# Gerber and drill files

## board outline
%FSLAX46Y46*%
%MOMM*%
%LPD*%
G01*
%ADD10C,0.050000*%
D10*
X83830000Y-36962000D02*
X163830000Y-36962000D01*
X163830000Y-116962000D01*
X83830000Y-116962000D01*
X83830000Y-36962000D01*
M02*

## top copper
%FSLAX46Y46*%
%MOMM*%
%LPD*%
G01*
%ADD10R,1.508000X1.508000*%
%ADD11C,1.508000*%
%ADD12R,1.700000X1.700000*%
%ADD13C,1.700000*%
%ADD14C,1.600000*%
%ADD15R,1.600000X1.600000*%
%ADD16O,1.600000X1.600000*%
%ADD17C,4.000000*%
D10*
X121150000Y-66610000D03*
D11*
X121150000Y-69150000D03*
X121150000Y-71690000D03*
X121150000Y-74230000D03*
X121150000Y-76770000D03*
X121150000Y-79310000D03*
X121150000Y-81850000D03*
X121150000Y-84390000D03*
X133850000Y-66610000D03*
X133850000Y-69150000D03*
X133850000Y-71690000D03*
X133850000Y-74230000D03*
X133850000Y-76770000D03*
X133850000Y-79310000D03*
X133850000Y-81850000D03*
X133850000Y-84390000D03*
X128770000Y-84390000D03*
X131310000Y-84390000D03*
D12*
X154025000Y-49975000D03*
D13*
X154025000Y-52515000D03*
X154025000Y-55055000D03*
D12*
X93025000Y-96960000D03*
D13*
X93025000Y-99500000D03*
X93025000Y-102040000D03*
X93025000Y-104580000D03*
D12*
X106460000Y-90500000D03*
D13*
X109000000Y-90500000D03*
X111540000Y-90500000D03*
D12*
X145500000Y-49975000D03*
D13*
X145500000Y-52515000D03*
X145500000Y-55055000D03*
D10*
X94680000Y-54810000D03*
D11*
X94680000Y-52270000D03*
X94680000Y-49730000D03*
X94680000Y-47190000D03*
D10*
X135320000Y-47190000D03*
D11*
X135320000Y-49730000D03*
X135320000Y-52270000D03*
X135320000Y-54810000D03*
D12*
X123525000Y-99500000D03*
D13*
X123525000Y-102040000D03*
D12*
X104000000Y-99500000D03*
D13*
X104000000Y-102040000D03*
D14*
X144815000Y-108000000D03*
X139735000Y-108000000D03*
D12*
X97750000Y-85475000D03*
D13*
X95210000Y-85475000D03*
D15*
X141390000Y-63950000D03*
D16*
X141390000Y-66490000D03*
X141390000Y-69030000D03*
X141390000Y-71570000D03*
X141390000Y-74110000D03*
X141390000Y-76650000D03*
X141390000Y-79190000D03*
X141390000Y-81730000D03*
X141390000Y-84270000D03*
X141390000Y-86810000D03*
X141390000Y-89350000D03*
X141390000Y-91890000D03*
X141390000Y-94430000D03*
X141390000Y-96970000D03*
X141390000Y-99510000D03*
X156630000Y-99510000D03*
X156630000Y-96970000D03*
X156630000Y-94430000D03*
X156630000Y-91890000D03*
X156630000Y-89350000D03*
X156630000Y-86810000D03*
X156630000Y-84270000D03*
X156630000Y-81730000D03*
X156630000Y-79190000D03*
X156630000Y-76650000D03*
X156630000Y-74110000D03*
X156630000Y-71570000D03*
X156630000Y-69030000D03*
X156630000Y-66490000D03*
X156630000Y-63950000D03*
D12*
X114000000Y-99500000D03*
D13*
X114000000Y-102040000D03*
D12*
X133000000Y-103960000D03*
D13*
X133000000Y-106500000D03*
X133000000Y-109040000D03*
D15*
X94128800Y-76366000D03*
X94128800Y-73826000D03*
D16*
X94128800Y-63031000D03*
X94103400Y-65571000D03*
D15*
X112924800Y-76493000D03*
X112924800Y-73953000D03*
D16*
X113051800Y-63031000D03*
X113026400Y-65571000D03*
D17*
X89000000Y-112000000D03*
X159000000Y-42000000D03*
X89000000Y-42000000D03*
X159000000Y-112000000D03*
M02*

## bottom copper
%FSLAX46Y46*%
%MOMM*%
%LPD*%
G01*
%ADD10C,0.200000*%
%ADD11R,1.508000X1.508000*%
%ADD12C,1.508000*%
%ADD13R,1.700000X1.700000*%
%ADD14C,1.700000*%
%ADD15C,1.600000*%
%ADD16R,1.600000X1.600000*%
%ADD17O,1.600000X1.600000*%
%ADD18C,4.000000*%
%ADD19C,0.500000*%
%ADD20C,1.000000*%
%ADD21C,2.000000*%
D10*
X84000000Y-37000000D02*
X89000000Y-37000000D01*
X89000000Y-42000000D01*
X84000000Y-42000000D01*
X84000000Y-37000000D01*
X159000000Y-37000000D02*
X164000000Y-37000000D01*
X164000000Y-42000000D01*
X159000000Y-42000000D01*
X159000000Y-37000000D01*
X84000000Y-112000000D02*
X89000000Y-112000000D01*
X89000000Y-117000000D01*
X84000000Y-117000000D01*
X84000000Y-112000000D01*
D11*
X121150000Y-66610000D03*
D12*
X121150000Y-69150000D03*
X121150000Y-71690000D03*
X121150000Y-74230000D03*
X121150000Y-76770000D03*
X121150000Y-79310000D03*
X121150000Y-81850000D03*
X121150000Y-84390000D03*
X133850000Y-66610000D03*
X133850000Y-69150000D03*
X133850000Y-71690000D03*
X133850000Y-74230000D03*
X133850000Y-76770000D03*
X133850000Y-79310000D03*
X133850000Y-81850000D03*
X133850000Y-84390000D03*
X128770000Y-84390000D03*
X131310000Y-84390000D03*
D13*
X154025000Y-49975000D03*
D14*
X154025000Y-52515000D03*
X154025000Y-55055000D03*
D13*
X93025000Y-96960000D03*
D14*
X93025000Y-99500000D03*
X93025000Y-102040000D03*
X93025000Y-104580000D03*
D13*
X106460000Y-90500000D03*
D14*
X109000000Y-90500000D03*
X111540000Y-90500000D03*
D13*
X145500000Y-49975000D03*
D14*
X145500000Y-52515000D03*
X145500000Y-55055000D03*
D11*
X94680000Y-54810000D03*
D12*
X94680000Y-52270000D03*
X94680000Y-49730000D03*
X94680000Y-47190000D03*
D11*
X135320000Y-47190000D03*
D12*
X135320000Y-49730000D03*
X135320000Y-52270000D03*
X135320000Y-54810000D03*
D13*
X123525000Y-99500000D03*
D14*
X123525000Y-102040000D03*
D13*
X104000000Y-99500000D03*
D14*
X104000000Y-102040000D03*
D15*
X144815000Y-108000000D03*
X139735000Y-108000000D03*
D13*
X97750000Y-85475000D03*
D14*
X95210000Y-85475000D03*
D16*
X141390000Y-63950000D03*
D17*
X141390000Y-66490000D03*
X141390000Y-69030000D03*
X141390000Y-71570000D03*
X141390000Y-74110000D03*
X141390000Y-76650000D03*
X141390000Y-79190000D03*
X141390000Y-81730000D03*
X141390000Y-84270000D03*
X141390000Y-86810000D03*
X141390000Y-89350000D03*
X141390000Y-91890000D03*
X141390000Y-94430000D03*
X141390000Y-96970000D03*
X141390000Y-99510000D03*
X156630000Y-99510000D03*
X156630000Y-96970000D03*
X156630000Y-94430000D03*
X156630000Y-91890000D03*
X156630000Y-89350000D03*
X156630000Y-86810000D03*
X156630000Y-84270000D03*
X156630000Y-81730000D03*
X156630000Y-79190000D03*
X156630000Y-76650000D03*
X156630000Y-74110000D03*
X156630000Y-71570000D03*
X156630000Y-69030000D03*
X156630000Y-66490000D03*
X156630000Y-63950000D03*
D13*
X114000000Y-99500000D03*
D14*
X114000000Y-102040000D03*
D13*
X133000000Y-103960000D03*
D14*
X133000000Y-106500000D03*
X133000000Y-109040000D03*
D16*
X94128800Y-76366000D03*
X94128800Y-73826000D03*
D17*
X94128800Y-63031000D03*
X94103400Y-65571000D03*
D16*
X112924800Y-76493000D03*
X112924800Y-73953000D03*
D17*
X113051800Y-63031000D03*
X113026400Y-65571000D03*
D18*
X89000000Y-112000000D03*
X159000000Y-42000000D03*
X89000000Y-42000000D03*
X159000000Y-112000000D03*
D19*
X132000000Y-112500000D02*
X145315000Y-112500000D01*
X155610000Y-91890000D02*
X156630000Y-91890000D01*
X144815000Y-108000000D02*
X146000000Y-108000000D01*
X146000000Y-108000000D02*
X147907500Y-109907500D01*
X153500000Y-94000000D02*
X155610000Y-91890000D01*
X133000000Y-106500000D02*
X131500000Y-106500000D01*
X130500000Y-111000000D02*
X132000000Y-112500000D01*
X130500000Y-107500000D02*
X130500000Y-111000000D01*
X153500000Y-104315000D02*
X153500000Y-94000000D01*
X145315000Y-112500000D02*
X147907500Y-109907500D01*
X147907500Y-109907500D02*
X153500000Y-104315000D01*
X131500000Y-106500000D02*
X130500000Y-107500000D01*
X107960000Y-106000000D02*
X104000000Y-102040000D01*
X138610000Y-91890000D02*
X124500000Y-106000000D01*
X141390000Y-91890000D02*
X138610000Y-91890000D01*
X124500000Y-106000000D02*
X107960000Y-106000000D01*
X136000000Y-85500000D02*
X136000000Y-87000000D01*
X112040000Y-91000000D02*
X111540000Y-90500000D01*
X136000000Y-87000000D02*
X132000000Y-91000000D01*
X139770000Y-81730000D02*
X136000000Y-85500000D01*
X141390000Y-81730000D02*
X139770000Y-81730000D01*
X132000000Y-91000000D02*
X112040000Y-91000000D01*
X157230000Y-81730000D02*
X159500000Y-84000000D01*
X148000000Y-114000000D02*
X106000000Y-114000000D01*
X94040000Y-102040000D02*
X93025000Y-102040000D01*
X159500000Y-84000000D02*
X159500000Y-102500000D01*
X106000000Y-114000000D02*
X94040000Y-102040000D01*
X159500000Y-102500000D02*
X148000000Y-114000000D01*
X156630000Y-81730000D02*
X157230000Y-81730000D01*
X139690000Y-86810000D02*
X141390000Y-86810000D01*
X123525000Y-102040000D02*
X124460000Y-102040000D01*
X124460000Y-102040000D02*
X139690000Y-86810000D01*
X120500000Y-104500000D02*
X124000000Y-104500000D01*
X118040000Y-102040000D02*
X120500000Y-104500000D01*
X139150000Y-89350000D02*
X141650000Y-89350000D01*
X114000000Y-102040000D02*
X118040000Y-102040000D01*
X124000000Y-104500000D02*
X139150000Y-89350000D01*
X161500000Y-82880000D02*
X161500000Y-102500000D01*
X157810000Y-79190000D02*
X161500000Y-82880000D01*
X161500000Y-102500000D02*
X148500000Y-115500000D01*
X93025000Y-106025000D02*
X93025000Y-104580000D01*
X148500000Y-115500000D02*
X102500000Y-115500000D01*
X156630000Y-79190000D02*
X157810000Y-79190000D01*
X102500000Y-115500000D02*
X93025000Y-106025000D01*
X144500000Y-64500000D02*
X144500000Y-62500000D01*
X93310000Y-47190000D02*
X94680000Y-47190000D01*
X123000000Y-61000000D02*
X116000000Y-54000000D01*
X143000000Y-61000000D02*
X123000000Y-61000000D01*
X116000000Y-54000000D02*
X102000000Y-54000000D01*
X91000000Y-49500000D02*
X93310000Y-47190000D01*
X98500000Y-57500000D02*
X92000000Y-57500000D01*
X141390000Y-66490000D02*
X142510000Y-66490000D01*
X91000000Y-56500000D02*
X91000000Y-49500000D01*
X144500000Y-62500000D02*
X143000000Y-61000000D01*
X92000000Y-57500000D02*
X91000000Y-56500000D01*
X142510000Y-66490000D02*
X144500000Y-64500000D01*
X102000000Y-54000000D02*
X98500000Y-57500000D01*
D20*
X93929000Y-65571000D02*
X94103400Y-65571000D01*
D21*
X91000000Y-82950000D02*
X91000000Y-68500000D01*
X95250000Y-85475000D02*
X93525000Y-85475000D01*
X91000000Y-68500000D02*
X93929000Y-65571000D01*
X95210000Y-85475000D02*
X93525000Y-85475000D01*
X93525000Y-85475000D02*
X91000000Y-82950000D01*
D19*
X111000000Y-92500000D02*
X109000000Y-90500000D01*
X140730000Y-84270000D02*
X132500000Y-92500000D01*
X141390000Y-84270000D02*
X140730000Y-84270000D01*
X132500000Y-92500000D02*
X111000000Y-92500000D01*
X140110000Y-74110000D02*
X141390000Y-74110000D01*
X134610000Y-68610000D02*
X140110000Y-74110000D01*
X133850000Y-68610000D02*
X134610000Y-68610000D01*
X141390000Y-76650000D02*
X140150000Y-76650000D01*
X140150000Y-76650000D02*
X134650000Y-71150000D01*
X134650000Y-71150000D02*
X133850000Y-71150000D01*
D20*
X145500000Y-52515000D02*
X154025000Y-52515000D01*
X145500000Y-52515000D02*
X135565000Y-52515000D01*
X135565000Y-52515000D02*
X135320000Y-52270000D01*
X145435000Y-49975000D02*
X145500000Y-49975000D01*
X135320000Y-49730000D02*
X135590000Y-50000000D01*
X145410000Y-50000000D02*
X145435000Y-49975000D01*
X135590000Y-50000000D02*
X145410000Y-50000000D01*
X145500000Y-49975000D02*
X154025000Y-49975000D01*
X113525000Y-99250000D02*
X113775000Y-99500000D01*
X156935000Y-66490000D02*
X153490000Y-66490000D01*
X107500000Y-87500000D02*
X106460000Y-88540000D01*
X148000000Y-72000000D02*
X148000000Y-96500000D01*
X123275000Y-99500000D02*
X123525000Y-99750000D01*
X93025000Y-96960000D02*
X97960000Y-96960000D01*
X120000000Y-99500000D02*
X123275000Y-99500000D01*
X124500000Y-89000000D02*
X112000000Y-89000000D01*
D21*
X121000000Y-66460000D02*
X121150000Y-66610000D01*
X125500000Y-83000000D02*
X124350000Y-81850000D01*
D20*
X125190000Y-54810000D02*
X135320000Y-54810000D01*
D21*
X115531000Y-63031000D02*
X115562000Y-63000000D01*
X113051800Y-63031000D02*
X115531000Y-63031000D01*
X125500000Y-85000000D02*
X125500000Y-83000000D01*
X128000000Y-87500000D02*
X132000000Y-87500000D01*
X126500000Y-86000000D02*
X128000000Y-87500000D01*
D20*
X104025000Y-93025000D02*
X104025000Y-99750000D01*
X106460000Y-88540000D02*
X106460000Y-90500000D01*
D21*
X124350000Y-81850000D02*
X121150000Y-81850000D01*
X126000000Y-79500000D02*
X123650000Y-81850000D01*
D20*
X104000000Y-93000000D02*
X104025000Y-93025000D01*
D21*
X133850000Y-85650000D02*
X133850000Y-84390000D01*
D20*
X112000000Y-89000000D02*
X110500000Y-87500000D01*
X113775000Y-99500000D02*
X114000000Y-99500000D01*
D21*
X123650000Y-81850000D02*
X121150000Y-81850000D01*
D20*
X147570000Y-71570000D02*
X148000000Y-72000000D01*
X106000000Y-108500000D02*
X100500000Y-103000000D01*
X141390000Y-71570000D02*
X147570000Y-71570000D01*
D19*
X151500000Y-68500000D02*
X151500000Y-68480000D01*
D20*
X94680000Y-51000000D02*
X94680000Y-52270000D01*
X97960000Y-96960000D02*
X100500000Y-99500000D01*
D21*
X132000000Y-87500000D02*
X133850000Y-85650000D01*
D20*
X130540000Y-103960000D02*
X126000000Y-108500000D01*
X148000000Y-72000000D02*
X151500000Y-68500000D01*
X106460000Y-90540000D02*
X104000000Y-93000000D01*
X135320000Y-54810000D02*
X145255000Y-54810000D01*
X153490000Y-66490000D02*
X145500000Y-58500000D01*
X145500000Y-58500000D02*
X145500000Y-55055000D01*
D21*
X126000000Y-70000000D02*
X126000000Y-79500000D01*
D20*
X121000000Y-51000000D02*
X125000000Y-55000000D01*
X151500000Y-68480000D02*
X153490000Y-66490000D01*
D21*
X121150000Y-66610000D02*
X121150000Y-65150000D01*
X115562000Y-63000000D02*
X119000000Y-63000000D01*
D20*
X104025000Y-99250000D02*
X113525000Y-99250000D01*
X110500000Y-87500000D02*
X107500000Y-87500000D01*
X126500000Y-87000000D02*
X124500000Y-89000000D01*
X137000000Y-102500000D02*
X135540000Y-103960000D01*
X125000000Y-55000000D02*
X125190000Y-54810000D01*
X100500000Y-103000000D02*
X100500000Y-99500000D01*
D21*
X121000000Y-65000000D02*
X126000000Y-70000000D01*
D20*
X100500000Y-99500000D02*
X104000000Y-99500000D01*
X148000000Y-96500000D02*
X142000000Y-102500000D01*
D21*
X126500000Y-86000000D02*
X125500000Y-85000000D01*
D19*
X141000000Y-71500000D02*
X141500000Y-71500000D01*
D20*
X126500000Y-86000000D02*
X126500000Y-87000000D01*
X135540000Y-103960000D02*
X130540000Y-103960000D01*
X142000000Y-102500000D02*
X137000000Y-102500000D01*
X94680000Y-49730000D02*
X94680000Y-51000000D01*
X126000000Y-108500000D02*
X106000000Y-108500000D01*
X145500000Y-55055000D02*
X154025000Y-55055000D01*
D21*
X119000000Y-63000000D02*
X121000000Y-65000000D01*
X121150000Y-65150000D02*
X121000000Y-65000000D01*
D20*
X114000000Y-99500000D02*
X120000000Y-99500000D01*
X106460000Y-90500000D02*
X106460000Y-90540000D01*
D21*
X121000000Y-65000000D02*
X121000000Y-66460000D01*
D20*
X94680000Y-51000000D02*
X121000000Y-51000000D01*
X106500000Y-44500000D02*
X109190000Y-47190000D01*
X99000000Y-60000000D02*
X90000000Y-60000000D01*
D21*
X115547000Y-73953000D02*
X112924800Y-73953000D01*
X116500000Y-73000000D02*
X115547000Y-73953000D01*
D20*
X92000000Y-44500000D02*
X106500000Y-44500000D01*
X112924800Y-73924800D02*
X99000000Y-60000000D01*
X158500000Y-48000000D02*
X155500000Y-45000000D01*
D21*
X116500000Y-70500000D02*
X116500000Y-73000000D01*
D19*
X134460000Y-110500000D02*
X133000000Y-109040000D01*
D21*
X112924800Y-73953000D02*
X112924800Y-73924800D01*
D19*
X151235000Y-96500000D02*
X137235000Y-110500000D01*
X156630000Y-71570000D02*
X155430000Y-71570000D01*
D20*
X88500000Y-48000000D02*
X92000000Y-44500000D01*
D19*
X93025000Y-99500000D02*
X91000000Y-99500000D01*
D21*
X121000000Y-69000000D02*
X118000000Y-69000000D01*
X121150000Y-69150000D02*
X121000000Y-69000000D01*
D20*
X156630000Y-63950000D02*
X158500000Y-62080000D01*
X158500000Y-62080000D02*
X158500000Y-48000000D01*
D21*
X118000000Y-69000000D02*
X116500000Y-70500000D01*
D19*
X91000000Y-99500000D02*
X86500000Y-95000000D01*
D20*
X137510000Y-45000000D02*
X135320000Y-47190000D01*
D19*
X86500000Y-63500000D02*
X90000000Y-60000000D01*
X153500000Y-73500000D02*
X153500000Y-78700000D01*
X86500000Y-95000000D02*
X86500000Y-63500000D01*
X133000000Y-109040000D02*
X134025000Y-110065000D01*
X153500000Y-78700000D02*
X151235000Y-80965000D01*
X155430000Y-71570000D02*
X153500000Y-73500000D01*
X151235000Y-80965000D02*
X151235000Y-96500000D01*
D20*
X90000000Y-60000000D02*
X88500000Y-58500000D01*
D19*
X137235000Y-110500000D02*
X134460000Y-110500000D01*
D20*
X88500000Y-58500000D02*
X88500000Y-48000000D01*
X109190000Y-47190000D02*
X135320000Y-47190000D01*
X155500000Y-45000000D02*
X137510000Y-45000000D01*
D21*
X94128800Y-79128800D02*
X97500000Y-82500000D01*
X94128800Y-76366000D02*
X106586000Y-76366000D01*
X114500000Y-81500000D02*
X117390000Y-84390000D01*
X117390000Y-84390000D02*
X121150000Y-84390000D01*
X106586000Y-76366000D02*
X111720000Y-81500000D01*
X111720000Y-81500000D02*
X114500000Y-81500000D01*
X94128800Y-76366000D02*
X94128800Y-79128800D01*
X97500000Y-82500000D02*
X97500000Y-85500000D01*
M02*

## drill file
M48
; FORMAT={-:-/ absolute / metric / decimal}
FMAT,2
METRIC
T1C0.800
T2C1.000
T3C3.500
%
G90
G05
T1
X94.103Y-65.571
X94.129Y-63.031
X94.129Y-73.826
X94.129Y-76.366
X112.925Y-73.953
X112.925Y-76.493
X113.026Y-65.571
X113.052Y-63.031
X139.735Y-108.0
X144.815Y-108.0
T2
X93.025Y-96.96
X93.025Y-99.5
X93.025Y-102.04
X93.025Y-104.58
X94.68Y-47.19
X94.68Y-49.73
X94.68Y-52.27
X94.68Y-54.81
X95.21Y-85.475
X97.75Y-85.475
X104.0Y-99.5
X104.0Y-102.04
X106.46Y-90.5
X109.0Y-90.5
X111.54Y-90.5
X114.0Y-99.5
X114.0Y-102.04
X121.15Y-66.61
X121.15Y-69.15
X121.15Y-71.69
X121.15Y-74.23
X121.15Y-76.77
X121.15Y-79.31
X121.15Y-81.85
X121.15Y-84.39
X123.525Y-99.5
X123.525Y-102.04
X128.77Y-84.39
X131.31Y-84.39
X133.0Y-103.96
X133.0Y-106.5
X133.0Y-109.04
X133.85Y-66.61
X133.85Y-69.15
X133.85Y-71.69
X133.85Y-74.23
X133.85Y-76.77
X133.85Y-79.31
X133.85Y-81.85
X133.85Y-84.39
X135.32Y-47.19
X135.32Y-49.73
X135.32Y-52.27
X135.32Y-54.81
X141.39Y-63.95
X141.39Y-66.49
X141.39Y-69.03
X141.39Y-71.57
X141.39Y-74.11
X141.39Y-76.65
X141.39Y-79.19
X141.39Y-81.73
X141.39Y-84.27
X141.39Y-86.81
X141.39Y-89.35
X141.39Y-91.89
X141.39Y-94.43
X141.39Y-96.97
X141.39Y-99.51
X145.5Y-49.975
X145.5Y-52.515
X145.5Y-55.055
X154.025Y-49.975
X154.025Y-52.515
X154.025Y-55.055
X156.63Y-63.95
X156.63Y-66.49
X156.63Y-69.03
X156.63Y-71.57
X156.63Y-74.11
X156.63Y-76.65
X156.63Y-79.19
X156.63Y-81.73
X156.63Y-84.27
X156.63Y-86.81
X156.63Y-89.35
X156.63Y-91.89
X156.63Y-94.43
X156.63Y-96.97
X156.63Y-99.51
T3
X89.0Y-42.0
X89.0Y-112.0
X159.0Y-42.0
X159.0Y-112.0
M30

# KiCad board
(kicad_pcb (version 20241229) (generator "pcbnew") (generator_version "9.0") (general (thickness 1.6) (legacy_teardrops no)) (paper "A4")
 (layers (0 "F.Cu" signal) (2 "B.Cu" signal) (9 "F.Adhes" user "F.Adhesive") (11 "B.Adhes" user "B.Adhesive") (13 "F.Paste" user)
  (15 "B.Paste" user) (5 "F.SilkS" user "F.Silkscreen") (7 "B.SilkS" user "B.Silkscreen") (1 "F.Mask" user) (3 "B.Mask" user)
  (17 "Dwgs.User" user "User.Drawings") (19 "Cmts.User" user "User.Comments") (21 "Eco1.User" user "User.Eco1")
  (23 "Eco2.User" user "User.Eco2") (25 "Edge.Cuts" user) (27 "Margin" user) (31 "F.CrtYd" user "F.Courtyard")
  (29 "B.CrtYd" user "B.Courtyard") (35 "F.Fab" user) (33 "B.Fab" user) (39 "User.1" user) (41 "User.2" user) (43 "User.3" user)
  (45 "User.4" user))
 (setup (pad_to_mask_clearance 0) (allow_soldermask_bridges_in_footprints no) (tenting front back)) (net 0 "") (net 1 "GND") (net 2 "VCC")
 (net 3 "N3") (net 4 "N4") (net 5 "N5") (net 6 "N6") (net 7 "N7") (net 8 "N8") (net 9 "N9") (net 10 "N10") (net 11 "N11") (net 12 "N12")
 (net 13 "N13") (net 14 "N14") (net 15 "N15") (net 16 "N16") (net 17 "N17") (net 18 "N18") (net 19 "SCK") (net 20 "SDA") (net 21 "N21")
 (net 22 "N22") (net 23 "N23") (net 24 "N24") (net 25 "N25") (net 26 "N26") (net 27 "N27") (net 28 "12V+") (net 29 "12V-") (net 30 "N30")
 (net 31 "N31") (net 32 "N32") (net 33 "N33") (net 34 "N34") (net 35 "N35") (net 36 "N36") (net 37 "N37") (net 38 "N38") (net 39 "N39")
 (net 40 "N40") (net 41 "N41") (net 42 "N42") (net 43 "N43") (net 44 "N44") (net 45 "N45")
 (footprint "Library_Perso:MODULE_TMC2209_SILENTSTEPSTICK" (layer "F.Cu") (at 127.5 75.5)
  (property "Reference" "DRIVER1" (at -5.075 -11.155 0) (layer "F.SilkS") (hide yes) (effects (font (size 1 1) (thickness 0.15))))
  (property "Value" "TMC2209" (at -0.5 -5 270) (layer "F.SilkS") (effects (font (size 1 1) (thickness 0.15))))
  (pad "1" thru_hole rect (at -6.35 -8.89) (size 1.508 1.508) (drill 1) (layers "*.Cu" "*.Mask") (remove_unused_layers no) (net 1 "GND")
   (solder_mask_margin 0.102))
  (pad "2" thru_hole circle (at -6.35 -6.35) (size 1.508 1.508) (drill 1) (layers "*.Cu" "*.Mask") (remove_unused_layers no) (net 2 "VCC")
   (solder_mask_margin 0.102))
  (pad "3" thru_hole circle (at -6.35 -3.81) (size 1.508 1.508) (drill 1) (layers "*.Cu" "*.Mask") (remove_unused_layers no) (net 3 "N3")
   (solder_mask_margin 0.102))
  (pad "4" thru_hole circle (at -6.35 -1.27) (size 1.508 1.508) (drill 1) (layers "*.Cu" "*.Mask") (remove_unused_layers no) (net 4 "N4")
   (solder_mask_margin 0.102))
  (pad "5" thru_hole circle (at -6.35 1.27) (size 1.508 1.508) (drill 1) (layers "*.Cu" "*.Mask") (remove_unused_layers no) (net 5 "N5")
   (solder_mask_margin 0.102))
  (pad "6" thru_hole circle (at -6.35 3.81) (size 1.508 1.508) (drill 1) (layers "*.Cu" "*.Mask") (remove_unused_layers no) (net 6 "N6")
   (solder_mask_margin 0.102))
  (pad "7" thru_hole circle (at -6.35 6.35) (size 1.508 1.508) (drill 1) (layers "*.Cu" "*.Mask") (remove_unused_layers no) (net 1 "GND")
   (solder_mask_margin 0.102))
  (pad "8" thru_hole circle (at -6.35 8.89) (size 1.508 1.508) (drill 1) (layers "*.Cu" "*.Mask") (remove_unused_layers no) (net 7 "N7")
   (solder_mask_margin 0.102))
  (pad "9" thru_hole circle (at 6.35 -8.89) (size 1.508 1.508) (drill 1) (layers "*.Cu" "*.Mask") (remove_unused_layers no) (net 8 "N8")
   (solder_mask_margin 0.102))
  (pad "10" thru_hole circle (at 6.35 -6.35) (size 1.508 1.508) (drill 1) (layers "*.Cu" "*.Mask") (remove_unused_layers no) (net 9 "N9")
   (solder_mask_margin 0.102))
  (pad "11" thru_hole circle (at 6.35 -3.81) (size 1.508 1.508) (drill 1) (layers "*.Cu" "*.Mask") (remove_unused_layers no) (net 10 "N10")
   (solder_mask_margin 0.102))
  (pad "12" thru_hole circle (at 6.35 -1.27) (size 1.508 1.508) (drill 1) (layers "*.Cu" "*.Mask") (remove_unused_layers no) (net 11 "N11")
   (solder_mask_margin 0.102))
  (pad "13" thru_hole circle (at 6.35 1.27) (size 1.508 1.508) (drill 1) (layers "*.Cu" "*.Mask") (remove_unused_layers no) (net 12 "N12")
   (solder_mask_margin 0.102))
  (pad "14" thru_hole circle (at 6.35 3.81) (size 1.508 1.508) (drill 1) (layers "*.Cu" "*.Mask") (remove_unused_layers no) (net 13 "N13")
   (solder_mask_margin 0.102))
  (pad "15" thru_hole circle (at 6.35 6.35) (size 1.508 1.508) (drill 1) (layers "*.Cu" "*.Mask") (remove_unused_layers no) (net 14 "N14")
   (solder_mask_margin 0.102))
  (pad "16" thru_hole circle (at 6.35 8.89) (size 1.508 1.508) (drill 1) (layers "*.Cu" "*.Mask") (remove_unused_layers no) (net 1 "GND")
   (solder_mask_margin 0.102))
  (pad "17" thru_hole circle (at 1.27 8.89) (size 1.508 1.508) (drill 1) (layers "*.Cu" "*.Mask") (remove_unused_layers no) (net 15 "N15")
   (solder_mask_margin 0.102))
  (pad "18" thru_hole circle (at 3.81 8.89) (size 1.508 1.508) (drill 1) (layers "*.Cu" "*.Mask") (remove_unused_layers no) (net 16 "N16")
   (solder_mask_margin 0.102)))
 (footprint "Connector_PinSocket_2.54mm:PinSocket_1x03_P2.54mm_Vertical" (layer "F.Cu") (at 154.025 49.975)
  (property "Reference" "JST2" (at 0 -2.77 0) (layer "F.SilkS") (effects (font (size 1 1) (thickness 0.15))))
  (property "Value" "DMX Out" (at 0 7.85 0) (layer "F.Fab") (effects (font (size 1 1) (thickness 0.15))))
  (pad "1" thru_hole rect (at 0 0) (size 1.7 1.7) (drill 1) (layers "*.Cu" "*.Mask") (remove_unused_layers no) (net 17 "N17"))
  (pad "2" thru_hole circle (at 0 2.54) (size 1.7 1.7) (drill 1) (layers "*.Cu" "*.Mask") (remove_unused_layers no) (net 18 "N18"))
  (pad "3" thru_hole circle (at 0 5.08) (size 1.7 1.7) (drill 1) (layers "*.Cu" "*.Mask") (remove_unused_layers no) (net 1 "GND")))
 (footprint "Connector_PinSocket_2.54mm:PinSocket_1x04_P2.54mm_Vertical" (layer "F.Cu") (at 93.025 96.96)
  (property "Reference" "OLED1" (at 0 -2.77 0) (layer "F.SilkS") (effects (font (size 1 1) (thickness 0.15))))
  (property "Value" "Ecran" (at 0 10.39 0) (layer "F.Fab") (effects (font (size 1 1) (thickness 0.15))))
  (pad "1" thru_hole rect (at 0 0) (size 1.7 1.7) (drill 1) (layers "*.Cu" "*.Mask") (remove_unused_layers no) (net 1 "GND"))
  (pad "2" thru_hole circle (at 0 2.54) (size 1.7 1.7) (drill 1) (layers "*.Cu" "*.Mask") (remove_unused_layers no) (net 2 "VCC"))
  (pad "3" thru_hole circle (at 0 5.08) (size 1.7 1.7) (drill 1) (layers "*.Cu" "*.Mask") (remove_unused_layers no) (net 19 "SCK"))
  (pad "4" thru_hole circle (at 0 7.62) (size 1.7 1.7) (drill 1) (layers "*.Cu" "*.Mask") (remove_unused_layers no) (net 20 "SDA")))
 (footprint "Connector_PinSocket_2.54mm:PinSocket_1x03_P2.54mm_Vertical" (layer "F.Cu") (at 106.46 90.5 90)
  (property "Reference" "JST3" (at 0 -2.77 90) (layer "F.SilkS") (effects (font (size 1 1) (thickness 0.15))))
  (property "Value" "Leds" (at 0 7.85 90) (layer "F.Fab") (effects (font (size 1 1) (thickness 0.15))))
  (pad "1" thru_hole rect (at 0 0 90) (size 1.7 1.7) (drill 1) (layers "*.Cu" "*.Mask") (remove_unused_layers no) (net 1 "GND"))
  (pad "2" thru_hole circle (at 0 2.54 90) (size 1.7 1.7) (drill 1) (layers "*.Cu" "*.Mask") (remove_unused_layers no) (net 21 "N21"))
  (pad "3" thru_hole circle (at 0 5.08 90) (size 1.7 1.7) (drill 1) (layers "*.Cu" "*.Mask") (remove_unused_layers no) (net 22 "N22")))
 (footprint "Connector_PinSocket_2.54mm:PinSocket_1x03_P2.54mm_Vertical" (layer "F.Cu") (at 145.5 49.975)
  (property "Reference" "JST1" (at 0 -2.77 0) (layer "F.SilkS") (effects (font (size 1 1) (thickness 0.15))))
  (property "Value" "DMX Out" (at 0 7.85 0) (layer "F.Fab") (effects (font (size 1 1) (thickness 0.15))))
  (pad "1" thru_hole rect (at 0 0) (size 1.7 1.7) (drill 1) (layers "*.Cu" "*.Mask") (remove_unused_layers no) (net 17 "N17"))
  (pad "2" thru_hole circle (at 0 2.54) (size 1.7 1.7) (drill 1) (layers "*.Cu" "*.Mask") (remove_unused_layers no) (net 18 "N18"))
  (pad "3" thru_hole circle (at 0 5.08) (size 1.7 1.7) (drill 1) (layers "*.Cu" "*.Mask") (remove_unused_layers no) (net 1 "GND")))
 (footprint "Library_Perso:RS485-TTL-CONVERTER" (layer "F.Cu") (at 115 51)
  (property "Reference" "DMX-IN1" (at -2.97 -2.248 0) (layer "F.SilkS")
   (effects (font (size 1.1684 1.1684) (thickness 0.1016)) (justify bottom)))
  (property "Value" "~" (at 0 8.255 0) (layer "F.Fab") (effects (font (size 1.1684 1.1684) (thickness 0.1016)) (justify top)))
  (pad "J1.1" thru_hole rect (at -20.32 3.81) (size 1.508 1.508) (drill 1) (layers "*.Cu" "*.Mask") (remove_unused_layers no) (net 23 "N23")
   (solder_mask_margin 0.1016))
  (pad "J1.2" thru_hole circle (at -20.32 1.27) (size 1.508 1.508) (drill 1) (layers "*.Cu" "*.Mask") (remove_unused_layers no)
   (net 1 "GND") (solder_mask_margin 0.1016))
  (pad "J1.3" thru_hole circle (at -20.32 -1.27) (size 1.508 1.508) (drill 1) (layers "*.Cu" "*.Mask") (remove_unused_layers no)
   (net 1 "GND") (solder_mask_margin 0.1016))
  (pad "J1.4" thru_hole circle (at -20.32 -3.81) (size 1.508 1.508) (drill 1) (layers "*.Cu" "*.Mask") (remove_unused_layers no)
   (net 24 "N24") (solder_mask_margin 0.1016))
  (pad "J2.1" thru_hole rect (at 20.32 -3.81 180) (size 1.508 1.508) (drill 1) (layers "*.Cu" "*.Mask") (remove_unused_layers no)
   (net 2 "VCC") (solder_mask_margin 0.1016))
  (pad "J2.2" thru_hole circle (at 20.32 -1.27 180) (size 1.508 1.508) (drill 1) (layers "*.Cu" "*.Mask") (remove_unused_layers no)
   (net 17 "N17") (solder_mask_margin 0.1016))
  (pad "J2.3" thru_hole circle (at 20.32 1.27 180) (size 1.508 1.508) (drill 1) (layers "*.Cu" "*.Mask") (remove_unused_layers no)
   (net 18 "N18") (solder_mask_margin 0.1016))
  (pad "J2.4" thru_hole circle (at 20.32 3.81 180) (size 1.508 1.508) (drill 1) (layers "*.Cu" "*.Mask") (remove_unused_layers no)
   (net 1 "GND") (solder_mask_margin 0.1016)))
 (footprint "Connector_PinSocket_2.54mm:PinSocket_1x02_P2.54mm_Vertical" (layer "F.Cu") (at 123.525 99.5)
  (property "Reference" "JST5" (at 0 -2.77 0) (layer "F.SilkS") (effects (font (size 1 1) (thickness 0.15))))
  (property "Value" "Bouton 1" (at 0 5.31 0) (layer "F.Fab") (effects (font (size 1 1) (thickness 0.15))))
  (pad "1" thru_hole rect (at 0 0) (size 1.7 1.7) (drill 1) (layers "*.Cu" "*.Mask") (remove_unused_layers no) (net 1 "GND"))
  (pad "2" thru_hole circle (at 0 2.54) (size 1.7 1.7) (drill 1) (layers "*.Cu" "*.Mask") (remove_unused_layers no) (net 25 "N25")))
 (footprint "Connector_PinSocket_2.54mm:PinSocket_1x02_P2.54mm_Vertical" (layer "F.Cu") (at 104 99.5)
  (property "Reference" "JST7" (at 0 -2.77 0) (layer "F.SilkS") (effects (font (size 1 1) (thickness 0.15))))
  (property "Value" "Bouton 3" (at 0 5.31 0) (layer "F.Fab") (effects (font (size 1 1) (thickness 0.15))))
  (pad "1" thru_hole rect (at 0 0) (size 1.7 1.7) (drill 1) (layers "*.Cu" "*.Mask") (remove_unused_layers no) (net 1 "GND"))
  (pad "2" thru_hole circle (at 0 2.54) (size 1.7 1.7) (drill 1) (layers "*.Cu" "*.Mask") (remove_unused_layers no) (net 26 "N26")))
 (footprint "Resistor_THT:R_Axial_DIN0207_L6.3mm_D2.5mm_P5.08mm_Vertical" (layer "F.Cu") (at 144.815 108 180)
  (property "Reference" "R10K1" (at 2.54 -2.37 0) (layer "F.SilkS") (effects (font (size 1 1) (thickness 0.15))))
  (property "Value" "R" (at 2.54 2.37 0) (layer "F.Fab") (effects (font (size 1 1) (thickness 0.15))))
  (pad "1" thru_hole circle (at 0 0 180) (size 1.6 1.6) (drill 0.8) (layers "*.Cu" "*.Mask") (remove_unused_layers no) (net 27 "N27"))
  (pad "2" thru_hole circle (at 5.08 0 180) (size 1.6 1.6) (drill 0.8) (layers "*.Cu" "*.Mask") (remove_unused_layers no) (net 2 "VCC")))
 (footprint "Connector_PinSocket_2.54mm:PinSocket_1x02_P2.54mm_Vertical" (layer "F.Cu") (at 97.75 85.475 -90)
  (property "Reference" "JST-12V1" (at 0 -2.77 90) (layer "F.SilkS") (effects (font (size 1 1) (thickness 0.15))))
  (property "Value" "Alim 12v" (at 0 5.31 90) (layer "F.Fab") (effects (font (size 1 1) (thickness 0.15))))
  (pad "1" thru_hole rect (at 0 0 270) (size 1.7 1.7) (drill 1) (layers "*.Cu" "*.Mask") (remove_unused_layers no) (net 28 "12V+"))
  (pad "2" thru_hole circle (at 0 2.54 270) (size 1.7 1.7) (drill 1) (layers "*.Cu" "*.Mask") (remove_unused_layers no) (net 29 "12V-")))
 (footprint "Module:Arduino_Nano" (layer "F.Cu") (at 141.39 63.95)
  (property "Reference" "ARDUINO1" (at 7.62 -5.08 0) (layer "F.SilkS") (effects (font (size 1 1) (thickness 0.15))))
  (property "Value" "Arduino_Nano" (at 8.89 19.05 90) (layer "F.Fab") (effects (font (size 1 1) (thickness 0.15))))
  (pad "1" thru_hole rect (at 0 0) (size 1.6 1.6) (drill 1) (layers "*.Cu" "*.Mask") (remove_unused_layers no) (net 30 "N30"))
  (pad "2" thru_hole oval (at 0 2.54) (size 1.6 1.6) (drill 1) (layers "*.Cu" "*.Mask") (remove_unused_layers no) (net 24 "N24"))
  (pad "3" thru_hole oval (at 0 5.08) (size 1.6 1.6) (drill 1) (layers "*.Cu" "*.Mask") (remove_unused_layers no) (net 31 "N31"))
  (pad "4" thru_hole oval (at 0 7.62) (size 1.6 1.6) (drill 1) (layers "*.Cu" "*.Mask") (remove_unused_layers no) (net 1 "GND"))
  (pad "5" thru_hole oval (at 0 10.16) (size 1.6 1.6) (drill 1) (layers "*.Cu" "*.Mask") (remove_unused_layers no) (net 8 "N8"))
  (pad "6" thru_hole oval (at 0 12.7) (size 1.6 1.6) (drill 1) (layers "*.Cu" "*.Mask") (remove_unused_layers no) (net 9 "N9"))
  (pad "7" thru_hole oval (at 0 15.24) (size 1.6 1.6) (drill 1) (layers "*.Cu" "*.Mask") (remove_unused_layers no) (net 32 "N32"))
  (pad "8" thru_hole oval (at 0 17.78) (size 1.6 1.6) (drill 1) (layers "*.Cu" "*.Mask") (remove_unused_layers no) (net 22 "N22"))
  (pad "9" thru_hole oval (at 0 20.32) (size 1.6 1.6) (drill 1) (layers "*.Cu" "*.Mask") (remove_unused_layers no) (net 21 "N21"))
  (pad "10" thru_hole oval (at 0 22.86) (size 1.6 1.6) (drill 1) (layers "*.Cu" "*.Mask") (remove_unused_layers no) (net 25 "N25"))
  (pad "11" thru_hole oval (at 0 25.4) (size 1.6 1.6) (drill 1) (layers "*.Cu" "*.Mask") (remove_unused_layers no) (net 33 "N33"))
  (pad "12" thru_hole oval (at 0 27.94) (size 1.6 1.6) (drill 1) (layers "*.Cu" "*.Mask") (remove_unused_layers no) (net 26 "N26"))
  (pad "13" thru_hole oval (at 0 30.48) (size 1.6 1.6) (drill 1) (layers "*.Cu" "*.Mask") (remove_unused_layers no) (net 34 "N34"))
  (pad "14" thru_hole oval (at 0 33.02) (size 1.6 1.6) (drill 1) (layers "*.Cu" "*.Mask") (remove_unused_layers no) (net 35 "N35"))
  (pad "15" thru_hole oval (at 0 35.56) (size 1.6 1.6) (drill 1) (layers "*.Cu" "*.Mask") (remove_unused_layers no) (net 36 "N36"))
  (pad "16" thru_hole oval (at 15.24 35.56) (size 1.6 1.6) (drill 1) (layers "*.Cu" "*.Mask") (remove_unused_layers no) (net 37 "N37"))
  (pad "17" thru_hole oval (at 15.24 33.02) (size 1.6 1.6) (drill 1) (layers "*.Cu" "*.Mask") (remove_unused_layers no) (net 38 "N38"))
  (pad "18" thru_hole oval (at 15.24 30.48) (size 1.6 1.6) (drill 1) (layers "*.Cu" "*.Mask") (remove_unused_layers no) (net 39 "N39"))
  (pad "19" thru_hole oval (at 15.24 27.94) (size 1.6 1.6) (drill 1) (layers "*.Cu" "*.Mask") (remove_unused_layers no) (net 27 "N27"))
  (pad "20" thru_hole oval (at 15.24 25.4) (size 1.6 1.6) (drill 1) (layers "*.Cu" "*.Mask") (remove_unused_layers no) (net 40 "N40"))
  (pad "21" thru_hole oval (at 15.24 22.86) (size 1.6 1.6) (drill 1) (layers "*.Cu" "*.Mask") (remove_unused_layers no) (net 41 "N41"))
  (pad "22" thru_hole oval (at 15.24 20.32) (size 1.6 1.6) (drill 1) (layers "*.Cu" "*.Mask") (remove_unused_layers no) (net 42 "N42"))
  (pad "23" thru_hole oval (at 15.24 17.78) (size 1.6 1.6) (drill 1) (layers "*.Cu" "*.Mask") (remove_unused_layers no) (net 19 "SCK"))
  (pad "24" thru_hole oval (at 15.24 15.24) (size 1.6 1.6) (drill 1) (layers "*.Cu" "*.Mask") (remove_unused_layers no) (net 20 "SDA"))
  (pad "25" thru_hole oval (at 15.24 12.7) (size 1.6 1.6) (drill 1) (layers "*.Cu" "*.Mask") (remove_unused_layers no) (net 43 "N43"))
  (pad "26" thru_hole oval (at 15.24 10.16) (size 1.6 1.6) (drill 1) (layers "*.Cu" "*.Mask") (remove_unused_layers no) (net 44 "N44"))
  (pad "27" thru_hole oval (at 15.24 7.62) (size 1.6 1.6) (drill 1) (layers "*.Cu" "*.Mask") (remove_unused_layers no) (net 2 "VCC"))
  (pad "28" thru_hole oval (at 15.24 5.08) (size 1.6 1.6) (drill 1) (layers "*.Cu" "*.Mask") (remove_unused_layers no) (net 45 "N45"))
  (pad "29" thru_hole oval (at 15.24 2.54) (size 1.6 1.6) (drill 1) (layers "*.Cu" "*.Mask") (remove_unused_layers no) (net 1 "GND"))
  (pad "30" thru_hole oval (at 15.24 0) (size 1.6 1.6) (drill 1) (layers "*.Cu" "*.Mask") (remove_unused_layers no) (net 2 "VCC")))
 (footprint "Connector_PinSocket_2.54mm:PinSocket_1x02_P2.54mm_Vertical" (layer "F.Cu") (at 114 99.5)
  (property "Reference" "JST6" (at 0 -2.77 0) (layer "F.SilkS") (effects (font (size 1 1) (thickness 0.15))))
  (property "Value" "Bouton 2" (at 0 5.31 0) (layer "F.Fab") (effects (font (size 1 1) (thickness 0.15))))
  (pad "1" thru_hole rect (at 0 0) (size 1.7 1.7) (drill 1) (layers "*.Cu" "*.Mask") (remove_unused_layers no) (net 1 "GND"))
  (pad "2" thru_hole circle (at 0 2.54) (size 1.7 1.7) (drill 1) (layers "*.Cu" "*.Mask") (remove_unused_layers no) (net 33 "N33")))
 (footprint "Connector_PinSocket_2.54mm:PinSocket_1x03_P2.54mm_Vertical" (layer "F.Cu") (at 133 103.96)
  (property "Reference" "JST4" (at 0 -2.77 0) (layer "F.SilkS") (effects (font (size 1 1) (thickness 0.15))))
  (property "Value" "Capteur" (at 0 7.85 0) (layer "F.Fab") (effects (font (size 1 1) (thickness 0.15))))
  (pad "1" thru_hole rect (at 0 0) (size 1.7 1.7) (drill 1) (layers "*.Cu" "*.Mask") (remove_unused_layers no) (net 1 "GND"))
  (pad "2" thru_hole circle (at 0 2.54) (size 1.7 1.7) (drill 1) (layers "*.Cu" "*.Mask") (remove_unused_layers no) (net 27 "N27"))
  (pad "3" thru_hole circle (at 0 5.08) (size 1.7 1.7) (drill 1) (layers "*.Cu" "*.Mask") (remove_unused_layers no) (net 2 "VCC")))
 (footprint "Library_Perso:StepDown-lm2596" (layer "F.Cu") (at 105 69 180)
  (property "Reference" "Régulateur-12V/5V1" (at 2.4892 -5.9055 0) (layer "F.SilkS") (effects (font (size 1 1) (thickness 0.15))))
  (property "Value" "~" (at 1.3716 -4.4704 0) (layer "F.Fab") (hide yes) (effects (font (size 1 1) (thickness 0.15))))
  (pad "1" thru_hole rect (at 10.8712 -7.366 90) (size 1.6 1.6) (drill 0.8) (layers "*.Cu" "B.Mask") (remove_unused_layers no) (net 7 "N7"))
  (pad "1" thru_hole rect (at 10.8712 -4.826 90) (size 1.6 1.6) (drill 0.8) (layers "*.Cu" "B.Mask") (remove_unused_layers no) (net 7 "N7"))
  (pad "2" thru_hole oval (at 10.8712 5.969 90) (size 1.6 1.6) (drill 0.8) (layers "*.Cu" "B.Mask") (remove_unused_layers no)
   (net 29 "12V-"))
  (pad "2" thru_hole oval (at 10.8966 3.429 90) (size 1.6 1.6) (drill 0.8) (layers "*.Cu" "B.Mask") (remove_unused_layers no)
   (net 29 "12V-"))
  (pad "3" thru_hole rect (at -7.9248 -7.493 90) (size 1.6 1.6) (drill 0.8) (layers "*.Cu" "B.Mask") (remove_unused_layers no) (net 2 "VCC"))
  (pad "3" thru_hole rect (at -7.9248 -4.953 90) (size 1.6 1.6) (drill 0.8) (layers "*.Cu" "B.Mask") (remove_unused_layers no) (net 2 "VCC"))
  (pad "4" thru_hole oval (at -8.0518 5.969 90) (size 1.6 1.6) (drill 0.8) (layers "*.Cu" "B.Mask") (remove_unused_layers no) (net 1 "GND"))
  (pad "4" thru_hole oval (at -8.0264 3.429 90) (size 1.6 1.6) (drill 0.8) (layers "*.Cu" "B.Mask") (remove_unused_layers no) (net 1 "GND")))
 (gr_rect (start 84 37) (end 89 42) (stroke (width 0.2) (type solid)) (fill no) (layer "B.Cu"))
 (gr_rect (start 159 37) (end 164 42) (stroke (width 0.2) (type solid)) (fill no) (layer "B.Cu"))
 (gr_rect (start 84 112) (end 89 117) (stroke (width 0.2) (type solid)) (fill no) (layer "B.Cu"))
 (gr_rect (start 83.83 36.962) (end 163.83 116.962) (stroke (width 0.05) (type solid)) (fill no) (layer "Edge.Cuts"))
 (via (at 89 112) (size 4) (drill 3.5) (layers "F.Cu" "B.Cu") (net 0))
 (via (at 159 42) (size 4) (drill 3.5) (layers "F.Cu" "B.Cu") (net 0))
 (via (at 89 42) (size 4) (drill 3.5) (layers "F.Cu" "B.Cu") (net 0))
 (segment (start 132 112.5) (end 145.315 112.5) (width 0.5) (layer "B.Cu") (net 27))
 (segment (start 155.61 91.89) (end 156.63 91.89) (width 0.5) (layer "B.Cu") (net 27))
 (segment (start 144.815 108) (end 146 108) (width 0.5) (layer "B.Cu") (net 27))
 (segment (start 146 108) (end 147.9075 109.9075) (width 0.5) (layer "B.Cu") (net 27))
 (segment (start 153.5 94) (end 155.61 91.89) (width 0.5) (layer "B.Cu") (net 27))
 (segment (start 133 106.5) (end 131.5 106.5) (width 0.5) (layer "B.Cu") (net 27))
 (segment (start 130.5 111) (end 132 112.5) (width 0.5) (layer "B.Cu") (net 27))
 (segment (start 130.5 107.5) (end 130.5 111) (width 0.5) (layer "B.Cu") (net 27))
 (segment (start 153.5 104.315) (end 153.5 94) (width 0.5) (layer "B.Cu") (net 27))
 (segment (start 145.315 112.5) (end 147.9075 109.9075) (width 0.5) (layer "B.Cu") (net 27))
 (segment (start 147.9075 109.9075) (end 153.5 104.315) (width 0.5) (layer "B.Cu") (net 27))
 (segment (start 131.5 106.5) (end 130.5 107.5) (width 0.5) (layer "B.Cu") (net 27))
 (segment (start 107.96 106) (end 104 102.04) (width 0.5) (layer "B.Cu") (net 26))
 (segment (start 138.61 91.89) (end 124.5 106) (width 0.5) (layer "B.Cu") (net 26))
 (segment (start 141.39 91.89) (end 138.61 91.89) (width 0.5) (layer "B.Cu") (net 26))
 (segment (start 124.5 106) (end 107.96 106) (width 0.5) (layer "B.Cu") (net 26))
 (segment (start 136 85.5) (end 136 87) (width 0.5) (layer "B.Cu") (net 22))
 (segment (start 112.04 91) (end 111.54 90.5) (width 0.5) (layer "B.Cu") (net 22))
 (segment (start 136 87) (end 132 91) (width 0.5) (layer "B.Cu") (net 22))
 (segment (start 139.77 81.73) (end 136 85.5) (width 0.5) (layer "B.Cu") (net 22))
 (segment (start 141.39 81.73) (end 139.77 81.73) (width 0.5) (layer "B.Cu") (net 22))
 (segment (start 132 91) (end 112.04 91) (width 0.5) (layer "B.Cu") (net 22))
 (segment (start 157.23 81.73) (end 159.5 84) (width 0.5) (layer "B.Cu") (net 19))
 (segment (start 148 114) (end 106 114) (width 0.5) (layer "B.Cu") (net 19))
 (segment (start 94.04 102.04) (end 93.025 102.04) (width 0.5) (layer "B.Cu") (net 19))
 (segment (start 159.5 84) (end 159.5 102.5) (width 0.5) (layer "B.Cu") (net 19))
 (segment (start 106 114) (end 94.04 102.04) (width 0.5) (layer "B.Cu") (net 19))
 (segment (start 159.5 102.5) (end 148 114) (width 0.5) (layer "B.Cu") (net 19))
 (segment (start 156.63 81.73) (end 157.23 81.73) (width 0.5) (layer "B.Cu") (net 19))
 (segment (start 139.69 86.81) (end 141.39 86.81) (width 0.5) (layer "B.Cu") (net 25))
 (segment (start 123.525 102.04) (end 124.46 102.04) (width 0.5) (layer "B.Cu") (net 25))
 (segment (start 124.46 102.04) (end 139.69 86.81) (width 0.5) (layer "B.Cu") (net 25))
 (segment (start 120.5 104.5) (end 124 104.5) (width 0.5) (layer "B.Cu") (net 33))
 (segment (start 118.04 102.04) (end 120.5 104.5) (width 0.5) (layer "B.Cu") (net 33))
 (segment (start 139.15 89.35) (end 141.65 89.35) (width 0.5) (layer "B.Cu") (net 33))
 (segment (start 114 102.04) (end 118.04 102.04) (width 0.5) (layer "B.Cu") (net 33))
 (segment (start 124 104.5) (end 139.15 89.35) (width 0.5) (layer "B.Cu") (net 33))
 (via (at 159 112) (size 4) (drill 3.5) (layers "F.Cu" "B.Cu") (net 20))
 (segment (start 161.5 82.88) (end 161.5 102.5) (width 0.5) (layer "B.Cu") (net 20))
 (segment (start 157.81 79.19) (end 161.5 82.88) (width 0.5) (layer "B.Cu") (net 20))
 (segment (start 161.5 102.5) (end 148.5 115.5) (width 0.5) (layer "B.Cu") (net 20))
 (segment (start 93.025 106.025) (end 93.025 104.58) (width 0.5) (layer "B.Cu") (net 20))
 (segment (start 148.5 115.5) (end 102.5 115.5) (width 0.5) (layer "B.Cu") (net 20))
 (segment (start 156.63 79.19) (end 157.81 79.19) (width 0.5) (layer "B.Cu") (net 20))
 (segment (start 102.5 115.5) (end 93.025 106.025) (width 0.5) (layer "B.Cu") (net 20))
 (segment (start 144.5 64.5) (end 144.5 62.5) (width 0.5) (layer "B.Cu") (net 24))
 (segment (start 93.31 47.19) (end 94.68 47.19) (width 0.5) (layer "B.Cu") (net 24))
 (segment (start 123 61) (end 116 54) (width 0.5) (layer "B.Cu") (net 24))
 (segment (start 143 61) (end 123 61) (width 0.5) (layer "B.Cu") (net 24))
 (segment (start 116 54) (end 102 54) (width 0.5) (layer "B.Cu") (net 24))
 (segment (start 91 49.5) (end 93.31 47.19) (width 0.5) (layer "B.Cu") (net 24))
 (segment (start 98.5 57.5) (end 92 57.5) (width 0.5) (layer "B.Cu") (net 24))
 (segment (start 141.39 66.49) (end 142.51 66.49) (width 0.5) (layer "B.Cu") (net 24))
 (segment (start 91 56.5) (end 91 49.5) (width 0.5) (layer "B.Cu") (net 24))
 (segment (start 144.5 62.5) (end 143 61) (width 0.5) (layer "B.Cu") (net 24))
 (segment (start 92 57.5) (end 91 56.5) (width 0.5) (layer "B.Cu") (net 24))
 (segment (start 142.51 66.49) (end 144.5 64.5) (width 0.5) (layer "B.Cu") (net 24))
 (segment (start 102 54) (end 98.5 57.5) (width 0.5) (layer "B.Cu") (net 24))
 (segment (start 93.929 65.571) (end 94.1034 65.571) (width 1) (layer "B.Cu") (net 29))
 (segment (start 91 82.95) (end 91 68.5) (width 2) (layer "B.Cu") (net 29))
 (segment (start 95.25 85.475) (end 93.525 85.475) (width 2) (layer "B.Cu") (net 29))
 (segment (start 91 68.5) (end 93.929 65.571) (width 2) (layer "B.Cu") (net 29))
 (segment (start 95.21 85.475) (end 93.525 85.475) (width 2) (layer "B.Cu") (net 29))
 (segment (start 93.525 85.475) (end 91 82.95) (width 2) (layer "B.Cu") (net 29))
 (segment (start 111 92.5) (end 109 90.5) (width 0.5) (layer "B.Cu") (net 21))
 (segment (start 140.73 84.27) (end 132.5 92.5) (width 0.5) (layer "B.Cu") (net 21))
 (segment (start 141.39 84.27) (end 140.73 84.27) (width 0.5) (layer "B.Cu") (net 21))
 (segment (start 132.5 92.5) (end 111 92.5) (width 0.5) (layer "B.Cu") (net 21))
 (segment (start 140.11 74.11) (end 141.39 74.11) (width 0.5) (layer "B.Cu") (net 8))
 (segment (start 134.61 68.61) (end 140.11 74.11) (width 0.5) (layer "B.Cu") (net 8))
 (segment (start 133.85 68.61) (end 134.61 68.61) (width 0.5) (layer "B.Cu") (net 8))
 (segment (start 141.39 76.65) (end 140.15 76.65) (width 0.5) (layer "B.Cu") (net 9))
 (segment (start 140.15 76.65) (end 134.65 71.15) (width 0.5) (layer "B.Cu") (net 9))
 (segment (start 134.65 71.15) (end 133.85 71.15) (width 0.5) (layer "B.Cu") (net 9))
 (segment (start 145.5 52.515) (end 154.025 52.515) (width 1) (layer "B.Cu") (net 18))
 (segment (start 145.5 52.515) (end 135.565 52.515) (width 1) (layer "B.Cu") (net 18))
 (segment (start 135.565 52.515) (end 135.32 52.27) (width 1) (layer "B.Cu") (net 18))
 (segment (start 145.435 49.975) (end 145.5 49.975) (width 1) (layer "B.Cu") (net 17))
 (segment (start 135.32 49.73) (end 135.59 50) (width 1) (layer "B.Cu") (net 17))
 (segment (start 145.41 50) (end 145.435 49.975) (width 1) (layer "B.Cu") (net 17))
 (segment (start 135.59 50) (end 145.41 50) (width 1) (layer "B.Cu") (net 17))
 (segment (start 145.5 49.975) (end 154.025 49.975) (width 1) (layer "B.Cu") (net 17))
 (segment (start 113.525 99.25) (end 113.775 99.5) (width 1) (layer "B.Cu") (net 1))
 (segment (start 156.935 66.49) (end 153.49 66.49) (width 1) (layer "B.Cu") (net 1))
 (segment (start 107.5 87.5) (end 106.46 88.54) (width 1) (layer "B.Cu") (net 1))
 (segment (start 148 72) (end 148 96.5) (width 1) (layer "B.Cu") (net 1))
 (segment (start 123.275 99.5) (end 123.525 99.75) (width 1) (layer "B.Cu") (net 1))
 (segment (start 93.025 96.96) (end 97.96 96.96) (width 1) (layer "B.Cu") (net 1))
 (segment (start 120 99.5) (end 123.275 99.5) (width 1) (layer "B.Cu") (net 1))
 (segment (start 124.5 89) (end 112 89) (width 1) (layer "B.Cu") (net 1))
 (segment (start 121 66.46) (end 121.15 66.61) (width 2) (layer "B.Cu") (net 1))
 (segment (start 125.5 83) (end 124.35 81.85) (width 2) (layer "B.Cu") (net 1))
 (segment (start 125.19 54.81) (end 135.32 54.81) (width 1) (layer "B.Cu") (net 1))
 (segment (start 115.531 63.031) (end 115.562 63) (width 2) (layer "B.Cu") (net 1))
 (segment (start 113.0518 63.031) (end 115.531 63.031) (width 2) (layer "B.Cu") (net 1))
 (segment (start 125.5 85) (end 125.5 83) (width 2) (layer "B.Cu") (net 1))
 (segment (start 128 87.5) (end 132 87.5) (width 2) (layer "B.Cu") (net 1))
 (segment (start 126.5 86) (end 128 87.5) (width 2) (layer "B.Cu") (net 1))
 (segment (start 104.025 93.025) (end 104.025 99.75) (width 1) (layer "B.Cu") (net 1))
 (segment (start 106.46 88.54) (end 106.46 90.5) (width 1) (layer "B.Cu") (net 1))
 (segment (start 124.35 81.85) (end 121.15 81.85) (width 2) (layer "B.Cu") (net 1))
 (segment (start 126 79.5) (end 123.65 81.85) (width 2) (layer "B.Cu") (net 1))
 (segment (start 104 93) (end 104.025 93.025) (width 1) (layer "B.Cu") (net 1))
 (segment (start 133.85 85.65) (end 133.85 84.39) (width 2) (layer "B.Cu") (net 1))
 (segment (start 112 89) (end 110.5 87.5) (width 1) (layer "B.Cu") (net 1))
 (segment (start 113.775 99.5) (end 114 99.5) (width 1) (layer "B.Cu") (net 1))
 (segment (start 123.65 81.85) (end 121.15 81.85) (width 2) (layer "B.Cu") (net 1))
 (segment (start 147.57 71.57) (end 148 72) (width 1) (layer "B.Cu") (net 1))
 (segment (start 106 108.5) (end 100.5 103) (width 1) (layer "B.Cu") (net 1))
 (segment (start 141.39 71.57) (end 147.57 71.57) (width 1) (layer "B.Cu") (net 1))
 (segment (start 151.5 68.5) (end 151.5 68.48) (width 0.5) (layer "B.Cu") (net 1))
 (segment (start 94.68 51) (end 94.68 52.27) (width 1) (layer "B.Cu") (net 1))
 (segment (start 97.96 96.96) (end 100.5 99.5) (width 1) (layer "B.Cu") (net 1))
 (segment (start 132 87.5) (end 133.85 85.65) (width 2) (layer "B.Cu") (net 1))
 (segment (start 130.54 103.96) (end 126 108.5) (width 1) (layer "B.Cu") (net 1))
 (segment (start 148 72) (end 151.5 68.5) (width 1) (layer "B.Cu") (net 1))
 (segment (start 106.46 90.54) (end 104 93) (width 1) (layer "B.Cu") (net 1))
 (segment (start 135.32 54.81) (end 145.255 54.81) (width 1) (layer "B.Cu") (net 1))
 (segment (start 153.49 66.49) (end 145.5 58.5) (width 1) (layer "B.Cu") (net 1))
 (segment (start 145.5 58.5) (end 145.5 55.055) (width 1) (layer "B.Cu") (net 1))
 (segment (start 126 70) (end 126 79.5) (width 2) (layer "B.Cu") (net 1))
 (segment (start 121 51) (end 125 55) (width 1) (layer "B.Cu") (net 1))
 (segment (start 151.5 68.48) (end 153.49 66.49) (width 1) (layer "B.Cu") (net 1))
 (segment (start 121.15 66.61) (end 121.15 65.15) (width 2) (layer "B.Cu") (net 1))
 (segment (start 115.562 63) (end 119 63) (width 2) (layer "B.Cu") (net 1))
 (segment (start 104.025 99.25) (end 113.525 99.25) (width 1) (layer "B.Cu") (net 1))
 (segment (start 110.5 87.5) (end 107.5 87.5) (width 1) (layer "B.Cu") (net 1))
 (segment (start 126.5 87) (end 124.5 89) (width 1) (layer "B.Cu") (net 1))
 (segment (start 137 102.5) (end 135.54 103.96) (width 1) (layer "B.Cu") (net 1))
 (segment (start 125 55) (end 125.19 54.81) (width 1) (layer "B.Cu") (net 1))
 (segment (start 100.5 103) (end 100.5 99.5) (width 1) (layer "B.Cu") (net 1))
 (segment (start 121 65) (end 126 70) (width 2) (layer "B.Cu") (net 1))
 (segment (start 100.5 99.5) (end 104 99.5) (width 1) (layer "B.Cu") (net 1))
 (segment (start 148 96.5) (end 142 102.5) (width 1) (layer "B.Cu") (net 1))
 (segment (start 126.5 86) (end 125.5 85) (width 2) (layer "B.Cu") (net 1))
 (segment (start 141 71.5) (end 141.5 71.5) (width 0.5) (layer "B.Cu") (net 1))
 (segment (start 126.5 86) (end 126.5 87) (width 1) (layer "B.Cu") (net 1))
 (segment (start 135.54 103.96) (end 130.54 103.96) (width 1) (layer "B.Cu") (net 1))
 (segment (start 142 102.5) (end 137 102.5) (width 1) (layer "B.Cu") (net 1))
 (segment (start 94.68 49.73) (end 94.68 51) (width 1) (layer "B.Cu") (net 1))
 (segment (start 126 108.5) (end 106 108.5) (width 1) (layer "B.Cu") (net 1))
 (segment (start 145.5 55.055) (end 154.025 55.055) (width 1) (layer "B.Cu") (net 1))
 (segment (start 119 63) (end 121 65) (width 2) (layer "B.Cu") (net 1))
 (segment (start 121.15 65.15) (end 121 65) (width 2) (layer "B.Cu") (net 1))
 (segment (start 114 99.5) (end 120 99.5) (width 1) (layer "B.Cu") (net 1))
 (segment (start 106.46 90.5) (end 106.46 90.54) (width 1) (layer "B.Cu") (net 1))
 (segment (start 121 65) (end 121 66.46) (width 2) (layer "B.Cu") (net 1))
 (segment (start 94.68 51) (end 121 51) (width 1) (layer "B.Cu") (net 1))
 (segment (start 106.5 44.5) (end 109.19 47.19) (width 1) (layer "B.Cu") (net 2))
 (segment (start 99 60) (end 90 60) (width 1) (layer "B.Cu") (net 2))
 (segment (start 115.547 73.953) (end 112.9248 73.953) (width 2) (layer "B.Cu") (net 2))
 (segment (start 116.5 73) (end 115.547 73.953) (width 2) (layer "B.Cu") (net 2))
 (segment (start 92 44.5) (end 106.5 44.5) (width 1) (layer "B.Cu") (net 2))
 (segment (start 112.9248 73.9248) (end 99 60) (width 1) (layer "B.Cu") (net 2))
 (segment (start 158.5 48) (end 155.5 45) (width 1) (layer "B.Cu") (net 2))
 (segment (start 116.5 70.5) (end 116.5 73) (width 2) (layer "B.Cu") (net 2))
 (segment (start 134.46 110.5) (end 133 109.04) (width 0.5) (layer "B.Cu") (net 2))
 (segment (start 112.9248 73.953) (end 112.9248 73.9248) (width 2) (layer "B.Cu") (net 2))
 (segment (start 151.235 96.5) (end 137.235 110.5) (width 0.5) (layer "B.Cu") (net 2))
 (segment (start 156.63 71.57) (end 155.43 71.57) (width 0.5) (layer "B.Cu") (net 2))
 (segment (start 88.5 48) (end 92 44.5) (width 1) (layer "B.Cu") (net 2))
 (segment (start 93.025 99.5) (end 91 99.5) (width 0.5) (layer "B.Cu") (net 2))
 (segment (start 121 69) (end 118 69) (width 2) (layer "B.Cu") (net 2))
 (segment (start 121.15 69.15) (end 121 69) (width 2) (layer "B.Cu") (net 2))
 (segment (start 156.63 63.95) (end 158.5 62.08) (width 1) (layer "B.Cu") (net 2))
 (segment (start 158.5 62.08) (end 158.5 48) (width 1) (layer "B.Cu") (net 2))
 (segment (start 118 69) (end 116.5 70.5) (width 2) (layer "B.Cu") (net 2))
 (segment (start 91 99.5) (end 86.5 95) (width 0.5) (layer "B.Cu") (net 2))
 (segment (start 137.51 45) (end 135.32 47.19) (width 1) (layer "B.Cu") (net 2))
 (segment (start 86.5 63.5) (end 90 60) (width 0.5) (layer "B.Cu") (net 2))
 (segment (start 153.5 73.5) (end 153.5 78.7) (width 0.5) (layer "B.Cu") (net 2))
 (segment (start 86.5 95) (end 86.5 63.5) (width 0.5) (layer "B.Cu") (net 2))
 (segment (start 133 109.04) (end 134.025 110.065) (width 0.5) (layer "B.Cu") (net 2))
 (segment (start 153.5 78.7) (end 151.235 80.965) (width 0.5) (layer "B.Cu") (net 2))
 (segment (start 155.43 71.57) (end 153.5 73.5) (width 0.5) (layer "B.Cu") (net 2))
 (segment (start 151.235 80.965) (end 151.235 96.5) (width 0.5) (layer "B.Cu") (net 2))
 (segment (start 90 60) (end 88.5 58.5) (width 1) (layer "B.Cu") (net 2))
 (segment (start 137.235 110.5) (end 134.46 110.5) (width 0.5) (layer "B.Cu") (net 2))
 (segment (start 88.5 58.5) (end 88.5 48) (width 1) (layer "B.Cu") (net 2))
 (segment (start 109.19 47.19) (end 135.32 47.19) (width 1) (layer "B.Cu") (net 2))
 (segment (start 155.5 45) (end 137.51 45) (width 1) (layer "B.Cu") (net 2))
 (segment (start 94.1288 79.1288) (end 97.5 82.5) (width 2) (layer "B.Cu") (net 7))
 (segment (start 94.1288 76.366) (end 106.586 76.366) (width 2) (layer "B.Cu") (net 7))
 (segment (start 114.5 81.5) (end 117.39 84.39) (width 2) (layer "B.Cu") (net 7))
 (segment (start 117.39 84.39) (end 121.15 84.39) (width 2) (layer "B.Cu") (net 7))
 (segment (start 106.586 76.366) (end 111.72 81.5) (width 2) (layer "B.Cu") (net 7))
 (segment (start 111.72 81.5) (end 114.5 81.5) (width 2) (layer "B.Cu") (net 7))
 (segment (start 94.1288 76.366) (end 94.1288 79.1288) (width 2) (layer "B.Cu") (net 7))
 (segment (start 97.5 82.5) (end 97.5 85.5) (width 2) (layer "B.Cu") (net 7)))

